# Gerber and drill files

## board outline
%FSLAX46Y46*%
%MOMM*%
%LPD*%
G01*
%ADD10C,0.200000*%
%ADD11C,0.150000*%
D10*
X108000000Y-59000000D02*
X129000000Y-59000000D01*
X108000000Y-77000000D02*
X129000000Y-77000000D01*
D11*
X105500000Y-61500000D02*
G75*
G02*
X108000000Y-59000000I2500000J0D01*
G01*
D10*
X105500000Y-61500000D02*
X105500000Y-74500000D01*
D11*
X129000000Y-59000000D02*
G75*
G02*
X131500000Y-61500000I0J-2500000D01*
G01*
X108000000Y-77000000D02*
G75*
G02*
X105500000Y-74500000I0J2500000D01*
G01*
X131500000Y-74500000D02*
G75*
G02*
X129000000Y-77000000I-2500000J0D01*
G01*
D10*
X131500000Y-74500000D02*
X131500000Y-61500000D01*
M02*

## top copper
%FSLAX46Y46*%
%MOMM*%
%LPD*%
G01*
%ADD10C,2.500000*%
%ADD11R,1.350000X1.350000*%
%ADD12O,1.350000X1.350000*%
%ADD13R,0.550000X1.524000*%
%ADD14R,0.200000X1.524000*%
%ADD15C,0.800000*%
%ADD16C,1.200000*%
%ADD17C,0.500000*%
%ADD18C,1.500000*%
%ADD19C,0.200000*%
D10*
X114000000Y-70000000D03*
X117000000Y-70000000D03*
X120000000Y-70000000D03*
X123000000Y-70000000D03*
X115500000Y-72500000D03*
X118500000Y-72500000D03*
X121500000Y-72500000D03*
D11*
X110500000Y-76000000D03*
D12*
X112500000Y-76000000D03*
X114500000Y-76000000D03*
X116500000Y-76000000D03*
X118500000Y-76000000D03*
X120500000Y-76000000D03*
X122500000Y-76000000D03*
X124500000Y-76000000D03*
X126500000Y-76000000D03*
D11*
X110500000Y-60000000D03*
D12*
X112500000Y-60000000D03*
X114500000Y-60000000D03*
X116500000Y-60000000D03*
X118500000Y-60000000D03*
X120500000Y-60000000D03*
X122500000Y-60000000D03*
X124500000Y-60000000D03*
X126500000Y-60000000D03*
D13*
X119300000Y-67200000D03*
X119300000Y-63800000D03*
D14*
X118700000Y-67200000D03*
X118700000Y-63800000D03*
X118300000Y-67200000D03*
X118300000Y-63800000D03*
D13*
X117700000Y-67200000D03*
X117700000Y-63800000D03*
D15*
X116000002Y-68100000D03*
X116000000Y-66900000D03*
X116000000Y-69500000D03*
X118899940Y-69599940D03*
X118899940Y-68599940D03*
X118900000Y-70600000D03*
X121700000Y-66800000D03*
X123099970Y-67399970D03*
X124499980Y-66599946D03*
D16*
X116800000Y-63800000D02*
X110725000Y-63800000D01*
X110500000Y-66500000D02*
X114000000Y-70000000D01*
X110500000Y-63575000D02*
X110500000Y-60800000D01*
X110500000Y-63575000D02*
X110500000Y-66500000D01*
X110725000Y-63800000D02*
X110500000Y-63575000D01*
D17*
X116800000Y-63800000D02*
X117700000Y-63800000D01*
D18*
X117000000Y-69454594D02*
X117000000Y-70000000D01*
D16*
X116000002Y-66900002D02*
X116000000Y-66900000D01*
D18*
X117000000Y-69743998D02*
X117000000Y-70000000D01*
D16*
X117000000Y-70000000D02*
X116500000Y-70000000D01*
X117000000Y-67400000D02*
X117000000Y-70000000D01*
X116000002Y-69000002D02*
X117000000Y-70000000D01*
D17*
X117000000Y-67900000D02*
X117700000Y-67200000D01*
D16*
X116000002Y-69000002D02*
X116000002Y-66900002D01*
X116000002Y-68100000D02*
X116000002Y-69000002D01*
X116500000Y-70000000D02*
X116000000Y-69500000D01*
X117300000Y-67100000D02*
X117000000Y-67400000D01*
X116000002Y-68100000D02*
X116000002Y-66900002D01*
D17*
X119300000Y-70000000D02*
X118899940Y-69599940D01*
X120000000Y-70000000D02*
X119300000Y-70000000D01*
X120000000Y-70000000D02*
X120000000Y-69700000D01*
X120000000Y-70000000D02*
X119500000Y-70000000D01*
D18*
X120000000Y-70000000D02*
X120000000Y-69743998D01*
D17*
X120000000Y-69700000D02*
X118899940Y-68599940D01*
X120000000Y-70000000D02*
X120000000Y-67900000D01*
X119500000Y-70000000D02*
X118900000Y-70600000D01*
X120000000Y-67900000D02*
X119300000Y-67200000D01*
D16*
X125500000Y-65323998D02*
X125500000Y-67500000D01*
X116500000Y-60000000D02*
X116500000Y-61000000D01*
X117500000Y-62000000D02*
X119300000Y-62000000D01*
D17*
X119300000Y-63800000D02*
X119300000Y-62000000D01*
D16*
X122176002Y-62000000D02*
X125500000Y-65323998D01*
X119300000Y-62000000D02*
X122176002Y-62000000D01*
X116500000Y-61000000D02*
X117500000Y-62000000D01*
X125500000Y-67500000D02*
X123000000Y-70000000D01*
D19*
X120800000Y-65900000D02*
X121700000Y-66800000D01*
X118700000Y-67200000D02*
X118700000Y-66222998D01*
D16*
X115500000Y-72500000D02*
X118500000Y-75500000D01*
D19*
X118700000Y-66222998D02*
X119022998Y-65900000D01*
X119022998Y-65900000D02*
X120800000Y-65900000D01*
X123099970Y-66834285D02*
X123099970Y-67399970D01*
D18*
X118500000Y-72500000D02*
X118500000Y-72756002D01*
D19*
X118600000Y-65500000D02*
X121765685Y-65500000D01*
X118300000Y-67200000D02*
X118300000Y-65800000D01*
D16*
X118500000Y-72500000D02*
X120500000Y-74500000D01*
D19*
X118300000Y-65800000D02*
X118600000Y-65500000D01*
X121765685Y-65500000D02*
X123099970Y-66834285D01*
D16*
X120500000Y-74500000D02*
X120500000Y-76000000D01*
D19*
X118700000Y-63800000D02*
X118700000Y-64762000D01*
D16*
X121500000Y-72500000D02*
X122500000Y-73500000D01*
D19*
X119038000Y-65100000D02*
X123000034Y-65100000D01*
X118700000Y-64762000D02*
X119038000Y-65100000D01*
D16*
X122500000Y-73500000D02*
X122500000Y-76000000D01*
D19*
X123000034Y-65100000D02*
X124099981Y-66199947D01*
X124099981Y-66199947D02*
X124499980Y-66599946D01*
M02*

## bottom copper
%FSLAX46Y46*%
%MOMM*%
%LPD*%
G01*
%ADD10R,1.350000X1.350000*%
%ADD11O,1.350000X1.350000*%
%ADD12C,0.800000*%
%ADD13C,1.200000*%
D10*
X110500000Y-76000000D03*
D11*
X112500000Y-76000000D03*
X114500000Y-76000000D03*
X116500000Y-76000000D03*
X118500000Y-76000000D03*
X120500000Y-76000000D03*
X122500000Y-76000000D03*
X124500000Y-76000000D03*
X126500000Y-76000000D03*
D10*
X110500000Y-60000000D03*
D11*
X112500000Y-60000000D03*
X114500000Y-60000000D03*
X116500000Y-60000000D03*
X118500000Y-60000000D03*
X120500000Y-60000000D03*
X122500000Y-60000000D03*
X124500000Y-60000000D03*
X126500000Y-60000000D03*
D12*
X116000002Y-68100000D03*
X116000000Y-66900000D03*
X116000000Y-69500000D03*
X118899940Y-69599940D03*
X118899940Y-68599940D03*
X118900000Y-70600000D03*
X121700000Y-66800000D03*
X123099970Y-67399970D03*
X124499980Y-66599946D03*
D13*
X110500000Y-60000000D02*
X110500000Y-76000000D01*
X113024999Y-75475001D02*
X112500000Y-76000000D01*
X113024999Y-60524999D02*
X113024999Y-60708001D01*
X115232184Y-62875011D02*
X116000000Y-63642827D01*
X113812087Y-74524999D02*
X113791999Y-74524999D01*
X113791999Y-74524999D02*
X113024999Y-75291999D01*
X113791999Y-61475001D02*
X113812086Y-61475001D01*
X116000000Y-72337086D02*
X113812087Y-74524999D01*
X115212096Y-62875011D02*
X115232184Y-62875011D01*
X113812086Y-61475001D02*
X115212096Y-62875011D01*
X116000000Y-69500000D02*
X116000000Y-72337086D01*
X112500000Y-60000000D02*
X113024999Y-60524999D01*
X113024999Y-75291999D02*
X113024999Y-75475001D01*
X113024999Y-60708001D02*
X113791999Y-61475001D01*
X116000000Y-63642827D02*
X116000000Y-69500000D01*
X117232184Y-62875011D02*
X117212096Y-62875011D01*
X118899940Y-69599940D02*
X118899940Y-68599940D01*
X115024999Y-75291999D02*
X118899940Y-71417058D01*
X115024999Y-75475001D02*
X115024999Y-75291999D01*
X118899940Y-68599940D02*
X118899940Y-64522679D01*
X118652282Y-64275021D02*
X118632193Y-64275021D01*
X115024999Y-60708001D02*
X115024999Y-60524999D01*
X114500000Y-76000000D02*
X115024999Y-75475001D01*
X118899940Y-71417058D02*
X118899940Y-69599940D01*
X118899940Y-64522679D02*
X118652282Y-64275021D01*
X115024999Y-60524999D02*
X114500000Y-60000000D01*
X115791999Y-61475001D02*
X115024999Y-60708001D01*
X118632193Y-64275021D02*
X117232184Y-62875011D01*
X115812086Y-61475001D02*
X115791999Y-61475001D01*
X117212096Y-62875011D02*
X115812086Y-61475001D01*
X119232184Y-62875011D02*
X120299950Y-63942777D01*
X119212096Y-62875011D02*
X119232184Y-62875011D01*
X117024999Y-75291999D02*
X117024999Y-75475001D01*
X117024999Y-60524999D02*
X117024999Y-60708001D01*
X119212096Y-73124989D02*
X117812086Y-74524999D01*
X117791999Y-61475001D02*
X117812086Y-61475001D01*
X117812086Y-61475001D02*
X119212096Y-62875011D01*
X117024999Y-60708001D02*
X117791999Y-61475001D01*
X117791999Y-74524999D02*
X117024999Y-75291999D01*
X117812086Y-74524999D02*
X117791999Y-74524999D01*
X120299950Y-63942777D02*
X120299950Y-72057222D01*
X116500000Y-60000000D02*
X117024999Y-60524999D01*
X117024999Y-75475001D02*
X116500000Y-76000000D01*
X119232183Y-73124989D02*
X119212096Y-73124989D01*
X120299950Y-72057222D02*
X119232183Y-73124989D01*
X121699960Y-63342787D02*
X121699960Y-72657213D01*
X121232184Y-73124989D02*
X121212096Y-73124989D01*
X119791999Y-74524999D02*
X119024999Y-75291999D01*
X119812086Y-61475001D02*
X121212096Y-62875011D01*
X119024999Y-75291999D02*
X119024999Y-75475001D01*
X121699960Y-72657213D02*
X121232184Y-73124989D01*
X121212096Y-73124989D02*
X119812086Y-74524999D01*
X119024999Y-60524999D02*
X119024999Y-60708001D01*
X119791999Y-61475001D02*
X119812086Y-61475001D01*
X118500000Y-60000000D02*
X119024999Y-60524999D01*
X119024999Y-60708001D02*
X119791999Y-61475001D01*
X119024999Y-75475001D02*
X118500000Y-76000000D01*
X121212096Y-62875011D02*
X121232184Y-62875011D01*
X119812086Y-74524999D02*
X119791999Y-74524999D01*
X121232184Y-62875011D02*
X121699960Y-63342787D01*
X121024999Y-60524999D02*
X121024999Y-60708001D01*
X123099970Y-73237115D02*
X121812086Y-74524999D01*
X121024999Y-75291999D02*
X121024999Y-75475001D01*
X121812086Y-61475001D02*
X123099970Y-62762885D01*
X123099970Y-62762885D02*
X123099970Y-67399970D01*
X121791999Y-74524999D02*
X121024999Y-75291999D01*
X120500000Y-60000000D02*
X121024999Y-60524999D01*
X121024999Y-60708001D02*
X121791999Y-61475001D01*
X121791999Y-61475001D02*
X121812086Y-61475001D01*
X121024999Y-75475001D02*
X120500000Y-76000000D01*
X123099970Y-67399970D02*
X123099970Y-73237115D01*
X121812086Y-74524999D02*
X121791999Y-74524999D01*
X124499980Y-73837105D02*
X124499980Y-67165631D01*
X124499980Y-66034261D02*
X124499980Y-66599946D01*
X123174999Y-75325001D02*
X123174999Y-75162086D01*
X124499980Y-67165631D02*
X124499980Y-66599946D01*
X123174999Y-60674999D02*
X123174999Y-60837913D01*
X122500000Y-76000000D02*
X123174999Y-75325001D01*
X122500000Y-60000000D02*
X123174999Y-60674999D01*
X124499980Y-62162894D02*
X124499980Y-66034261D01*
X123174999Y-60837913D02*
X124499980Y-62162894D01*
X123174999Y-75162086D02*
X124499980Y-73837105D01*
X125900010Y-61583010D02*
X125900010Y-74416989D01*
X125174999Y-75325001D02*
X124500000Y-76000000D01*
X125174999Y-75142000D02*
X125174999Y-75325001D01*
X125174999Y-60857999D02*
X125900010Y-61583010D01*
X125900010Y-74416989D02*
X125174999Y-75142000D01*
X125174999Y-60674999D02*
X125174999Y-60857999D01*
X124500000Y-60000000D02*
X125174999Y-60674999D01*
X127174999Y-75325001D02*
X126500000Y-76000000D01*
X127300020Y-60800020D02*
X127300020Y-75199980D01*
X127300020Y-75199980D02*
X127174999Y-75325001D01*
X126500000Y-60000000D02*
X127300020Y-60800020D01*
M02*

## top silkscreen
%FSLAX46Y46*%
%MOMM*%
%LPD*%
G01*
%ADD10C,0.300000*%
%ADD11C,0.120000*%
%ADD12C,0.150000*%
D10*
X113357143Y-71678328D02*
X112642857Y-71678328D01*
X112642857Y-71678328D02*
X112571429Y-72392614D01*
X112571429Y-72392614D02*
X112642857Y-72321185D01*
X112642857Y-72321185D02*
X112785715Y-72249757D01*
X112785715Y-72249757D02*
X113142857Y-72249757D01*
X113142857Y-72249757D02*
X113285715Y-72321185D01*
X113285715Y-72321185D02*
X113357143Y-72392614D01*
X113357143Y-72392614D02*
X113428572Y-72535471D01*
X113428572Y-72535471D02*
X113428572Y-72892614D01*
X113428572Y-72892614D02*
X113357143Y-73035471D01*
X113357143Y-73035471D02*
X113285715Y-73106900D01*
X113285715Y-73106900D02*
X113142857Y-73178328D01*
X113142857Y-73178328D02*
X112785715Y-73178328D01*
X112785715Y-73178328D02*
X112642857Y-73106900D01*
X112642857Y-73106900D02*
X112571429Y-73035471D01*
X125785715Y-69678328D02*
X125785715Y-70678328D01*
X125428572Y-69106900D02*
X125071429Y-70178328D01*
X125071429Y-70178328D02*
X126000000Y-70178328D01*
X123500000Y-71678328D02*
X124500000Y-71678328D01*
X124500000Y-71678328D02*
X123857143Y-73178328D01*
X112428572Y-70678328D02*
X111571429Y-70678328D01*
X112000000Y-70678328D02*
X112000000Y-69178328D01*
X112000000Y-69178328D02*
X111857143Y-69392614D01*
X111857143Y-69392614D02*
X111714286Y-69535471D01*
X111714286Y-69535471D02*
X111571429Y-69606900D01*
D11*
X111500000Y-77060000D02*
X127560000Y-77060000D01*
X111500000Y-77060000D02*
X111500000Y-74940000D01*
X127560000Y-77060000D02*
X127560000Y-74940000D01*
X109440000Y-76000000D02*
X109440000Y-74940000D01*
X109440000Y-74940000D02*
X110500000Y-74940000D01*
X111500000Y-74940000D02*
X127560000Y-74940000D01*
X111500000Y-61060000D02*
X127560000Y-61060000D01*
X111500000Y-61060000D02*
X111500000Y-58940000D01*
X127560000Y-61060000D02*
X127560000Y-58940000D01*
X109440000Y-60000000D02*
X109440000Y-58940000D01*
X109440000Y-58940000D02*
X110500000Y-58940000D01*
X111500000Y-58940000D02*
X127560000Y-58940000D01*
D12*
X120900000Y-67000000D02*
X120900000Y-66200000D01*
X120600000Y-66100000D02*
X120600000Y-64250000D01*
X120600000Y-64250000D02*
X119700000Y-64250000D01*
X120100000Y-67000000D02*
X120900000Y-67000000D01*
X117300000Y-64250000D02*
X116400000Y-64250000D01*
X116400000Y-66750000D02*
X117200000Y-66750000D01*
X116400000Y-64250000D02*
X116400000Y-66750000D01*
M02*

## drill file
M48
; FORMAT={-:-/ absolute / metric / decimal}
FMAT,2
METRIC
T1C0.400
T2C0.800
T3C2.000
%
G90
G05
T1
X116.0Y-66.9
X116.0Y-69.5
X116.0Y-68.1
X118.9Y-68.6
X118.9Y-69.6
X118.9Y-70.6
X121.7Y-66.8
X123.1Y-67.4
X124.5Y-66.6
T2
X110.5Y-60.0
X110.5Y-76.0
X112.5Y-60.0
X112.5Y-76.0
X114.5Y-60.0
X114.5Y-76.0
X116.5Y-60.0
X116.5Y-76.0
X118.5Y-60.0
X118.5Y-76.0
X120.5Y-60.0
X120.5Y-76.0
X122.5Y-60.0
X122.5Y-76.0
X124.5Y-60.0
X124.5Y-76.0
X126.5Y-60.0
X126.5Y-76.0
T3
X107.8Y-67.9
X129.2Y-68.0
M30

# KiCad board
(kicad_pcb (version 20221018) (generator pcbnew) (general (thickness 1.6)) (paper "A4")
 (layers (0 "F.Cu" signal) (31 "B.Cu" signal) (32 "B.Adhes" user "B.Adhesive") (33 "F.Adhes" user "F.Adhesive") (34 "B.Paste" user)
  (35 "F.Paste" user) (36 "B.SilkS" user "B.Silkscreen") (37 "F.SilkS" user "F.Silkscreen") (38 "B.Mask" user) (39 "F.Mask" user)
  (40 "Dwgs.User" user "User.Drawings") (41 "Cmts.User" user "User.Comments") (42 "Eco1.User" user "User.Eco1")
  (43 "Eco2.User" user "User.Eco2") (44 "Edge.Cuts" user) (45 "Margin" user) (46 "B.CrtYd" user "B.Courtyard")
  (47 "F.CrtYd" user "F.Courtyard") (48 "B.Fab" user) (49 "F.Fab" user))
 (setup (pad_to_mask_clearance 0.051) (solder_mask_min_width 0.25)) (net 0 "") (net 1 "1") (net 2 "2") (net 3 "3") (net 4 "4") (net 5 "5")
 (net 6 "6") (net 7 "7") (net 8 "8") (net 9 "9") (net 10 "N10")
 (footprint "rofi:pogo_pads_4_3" (layer "F.Cu") (at 118.5 70)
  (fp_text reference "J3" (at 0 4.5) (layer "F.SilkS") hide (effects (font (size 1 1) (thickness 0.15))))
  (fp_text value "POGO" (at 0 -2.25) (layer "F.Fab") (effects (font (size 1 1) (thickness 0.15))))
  (pad "1" smd circle (at -4.5 0) (size 2.5 2.5) (layers "F.Cu" "F.Paste" "F.Mask") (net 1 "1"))
  (pad "2" smd circle (at -1.5 0) (size 2.5 2.5) (layers "F.Cu" "F.Paste" "F.Mask") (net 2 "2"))
  (pad "3" smd circle (at 1.5 0) (size 2.5 2.5) (layers "F.Cu" "F.Paste" "F.Mask") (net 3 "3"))
  (pad "4" smd circle (at 4.5 0) (size 2.5 2.5) (layers "F.Cu" "F.Paste" "F.Mask") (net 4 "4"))
  (pad "5" smd circle (at -3 2.5) (size 2.5 2.5) (layers "F.Cu" "F.Paste" "F.Mask") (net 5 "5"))
  (pad "6" smd circle (at 0 2.5) (size 2.5 2.5) (layers "F.Cu" "F.Paste" "F.Mask") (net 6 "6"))
  (pad "7" smd circle (at 3 2.5) (size 2.5 2.5) (layers "F.Cu" "F.Paste" "F.Mask") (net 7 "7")))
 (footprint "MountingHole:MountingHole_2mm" (layer "F.Cu") (at 129.2 68)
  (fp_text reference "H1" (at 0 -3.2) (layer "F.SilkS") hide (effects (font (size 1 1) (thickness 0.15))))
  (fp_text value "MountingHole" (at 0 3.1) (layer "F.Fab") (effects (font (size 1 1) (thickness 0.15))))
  (pad "" np_thru_hole circle (at 0 0) (size 2 2) (drill 2) (layers "*.Cu" "*.Mask")))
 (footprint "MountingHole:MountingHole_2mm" (layer "F.Cu") (at 107.8 67.9)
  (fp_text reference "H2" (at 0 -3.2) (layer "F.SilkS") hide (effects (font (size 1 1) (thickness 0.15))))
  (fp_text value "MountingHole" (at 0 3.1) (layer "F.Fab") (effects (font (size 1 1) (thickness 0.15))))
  (pad "" np_thru_hole circle (at 0 0) (size 2 2) (drill 2) (layers "*.Cu" "*.Mask")))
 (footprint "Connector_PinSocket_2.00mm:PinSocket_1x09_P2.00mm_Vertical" (layer "F.Cu") (at 110.5 76 90)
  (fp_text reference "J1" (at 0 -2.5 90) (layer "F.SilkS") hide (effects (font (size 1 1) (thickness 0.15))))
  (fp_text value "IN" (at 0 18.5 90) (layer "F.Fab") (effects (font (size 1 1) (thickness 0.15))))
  (fp_line (start -1.06 1) (end -1.06 17.06) (stroke (width 0.12) (type solid)) (layer "F.SilkS"))
  (fp_line (start -1.06 1) (end 1.06 1) (stroke (width 0.12) (type solid)) (layer "F.SilkS"))
  (fp_line (start -1.06 17.06) (end 1.06 17.06) (stroke (width 0.12) (type solid)) (layer "F.SilkS"))
  (fp_line (start 0 -1.06) (end 1.06 -1.06) (stroke (width 0.12) (type solid)) (layer "F.SilkS"))
  (fp_line (start 1.06 -1.06) (end 1.06 0) (stroke (width 0.12) (type solid)) (layer "F.SilkS"))
  (fp_line (start 1.06 1) (end 1.06 17.06) (stroke (width 0.12) (type solid)) (layer "F.SilkS"))
  (pad "1" thru_hole rect (at 0 0 90) (size 1.35 1.35) (drill 0.8) (layers "*.Cu" "*.Mask") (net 1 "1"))
  (pad "2" thru_hole oval (at 0 2 90) (size 1.35 1.35) (drill 0.8) (layers "*.Cu" "*.Mask") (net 2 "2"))
  (pad "3" thru_hole oval (at 0 4 90) (size 1.35 1.35) (drill 0.8) (layers "*.Cu" "*.Mask") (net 3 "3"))
  (pad "4" thru_hole oval (at 0 6 90) (size 1.35 1.35) (drill 0.8) (layers "*.Cu" "*.Mask") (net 4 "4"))
  (pad "5" thru_hole oval (at 0 8 90) (size 1.35 1.35) (drill 0.8) (layers "*.Cu" "*.Mask") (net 5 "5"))
  (pad "6" thru_hole oval (at 0 10 90) (size 1.35 1.35) (drill 0.8) (layers "*.Cu" "*.Mask") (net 6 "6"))
  (pad "7" thru_hole oval (at 0 12 90) (size 1.35 1.35) (drill 0.8) (layers "*.Cu" "*.Mask") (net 7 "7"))
  (pad "8" thru_hole oval (at 0 14 90) (size 1.35 1.35) (drill 0.8) (layers "*.Cu" "*.Mask") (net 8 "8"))
  (pad "9" thru_hole oval (at 0 16 90) (size 1.35 1.35) (drill 0.8) (layers "*.Cu" "*.Mask") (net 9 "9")))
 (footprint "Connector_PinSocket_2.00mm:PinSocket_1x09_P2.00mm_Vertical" (layer "F.Cu") (at 110.5 60 90)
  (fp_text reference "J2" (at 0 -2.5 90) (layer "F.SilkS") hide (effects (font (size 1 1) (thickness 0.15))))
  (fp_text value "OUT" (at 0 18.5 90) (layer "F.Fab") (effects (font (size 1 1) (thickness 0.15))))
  (fp_line (start -1.06 1) (end -1.06 17.06) (stroke (width 0.12) (type solid)) (layer "F.SilkS"))
  (fp_line (start -1.06 1) (end 1.06 1) (stroke (width 0.12) (type solid)) (layer "F.SilkS"))
  (fp_line (start -1.06 17.06) (end 1.06 17.06) (stroke (width 0.12) (type solid)) (layer "F.SilkS"))
  (fp_line (start 0 -1.06) (end 1.06 -1.06) (stroke (width 0.12) (type solid)) (layer "F.SilkS"))
  (fp_line (start 1.06 -1.06) (end 1.06 0) (stroke (width 0.12) (type solid)) (layer "F.SilkS"))
  (fp_line (start 1.06 1) (end 1.06 17.06) (stroke (width 0.12) (type solid)) (layer "F.SilkS"))
  (pad "1" thru_hole rect (at 0 0 90) (size 1.35 1.35) (drill 0.8) (layers "*.Cu" "*.Mask") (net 1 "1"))
  (pad "2" thru_hole oval (at 0 2 90) (size 1.35 1.35) (drill 0.8) (layers "*.Cu" "*.Mask") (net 2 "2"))
  (pad "3" thru_hole oval (at 0 4 90) (size 1.35 1.35) (drill 0.8) (layers "*.Cu" "*.Mask") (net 3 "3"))
  (pad "4" thru_hole oval (at 0 6 90) (size 1.35 1.35) (drill 0.8) (layers "*.Cu" "*.Mask") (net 4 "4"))
  (pad "5" thru_hole oval (at 0 8 90) (size 1.35 1.35) (drill 0.8) (layers "*.Cu" "*.Mask") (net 5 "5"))
  (pad "6" thru_hole oval (at 0 10 90) (size 1.35 1.35) (drill 0.8) (layers "*.Cu" "*.Mask") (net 6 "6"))
  (pad "7" thru_hole oval (at 0 12 90) (size 1.35 1.35) (drill 0.8) (layers "*.Cu" "*.Mask") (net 7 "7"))
  (pad "8" thru_hole oval (at 0 14 90) (size 1.35 1.35) (drill 0.8) (layers "*.Cu" "*.Mask") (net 8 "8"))
  (pad "9" thru_hole oval (at 0 16 90) (size 1.35 1.35) (drill 0.8) (layers "*.Cu" "*.Mask") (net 9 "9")))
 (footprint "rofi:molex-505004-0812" (layer "F.Cu") (at 118.5 65.5 180)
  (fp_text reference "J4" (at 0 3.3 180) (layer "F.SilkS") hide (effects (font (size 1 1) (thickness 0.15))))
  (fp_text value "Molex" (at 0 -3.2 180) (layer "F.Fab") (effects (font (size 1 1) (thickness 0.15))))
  (fp_line (start -2.4 -1.5) (end -2.4 -0.7) (stroke (width 0.15) (type solid)) (layer "F.SilkS"))
  (fp_line (start -2.1 -0.6) (end -2.1 1.25) (stroke (width 0.15) (type solid)) (layer "F.SilkS"))
  (fp_line (start -2.1 1.25) (end -1.2 1.25) (stroke (width 0.15) (type solid)) (layer "F.SilkS"))
  (fp_line (start -1.6 -1.5) (end -2.4 -1.5) (stroke (width 0.15) (type solid)) (layer "F.SilkS"))
  (fp_line (start 1.2 1.25) (end 2.1 1.25) (stroke (width 0.15) (type solid)) (layer "F.SilkS"))
  (fp_line (start 2.1 -1.25) (end 1.3 -1.25) (stroke (width 0.15) (type solid)) (layer "F.SilkS"))
  (fp_line (start 2.1 1.25) (end 2.1 -1.25) (stroke (width 0.15) (type solid)) (layer "F.SilkS"))
  (pad "1" smd rect (at -0.8 -1.7 180) (size 0.55 1.524) (layers "F.Cu" "F.Paste" "F.Mask") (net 3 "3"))
  (pad "2" smd rect (at -0.8 1.7 180) (size 0.55 1.524) (layers "F.Cu" "F.Paste" "F.Mask") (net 4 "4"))
  (pad "3" smd rect (at -0.2 -1.7 180) (size 0.2 1.524) (layers "F.Cu" "F.Paste" "F.Mask") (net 5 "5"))
  (pad "4" smd rect (at -0.2 1.7 180) (size 0.2 1.524) (layers "F.Cu" "F.Paste" "F.Mask") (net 7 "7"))
  (pad "5" smd rect (at 0.2 -1.7 180) (size 0.2 1.524) (layers "F.Cu" "F.Paste" "F.Mask") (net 6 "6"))
  (pad "6" smd rect (at 0.2 1.7 180) (size 0.2 1.524) (layers "F.Cu" "F.Paste" "F.Mask") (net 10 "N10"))
  (pad "7" smd rect (at 0.8 -1.7 180) (size 0.55 1.524) (layers "F.Cu" "F.Paste" "F.Mask") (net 2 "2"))
  (pad "8" smd rect (at 0.8 1.7 180) (size 0.55 1.524) (layers "F.Cu" "F.Paste" "F.Mask") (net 1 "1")))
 (gr_line (start 108 59) (end 129 59) (stroke (width 0.2) (type solid)) (layer "Edge.Cuts"))
 (gr_line (start 108 77) (end 129 77) (stroke (width 0.2) (type solid)) (layer "Edge.Cuts"))
 (gr_arc (start 105.5 61.5) (mid 106.232233 59.732233) (end 108 59) (stroke (width 0.15) (type solid)) (layer "Edge.Cuts"))
 (gr_line (start 105.5 61.5) (end 105.5 74.5) (stroke (width 0.2) (type solid)) (layer "Edge.Cuts"))
 (gr_arc (start 129 59) (mid 130.767767 59.732233) (end 131.5 61.5) (stroke (width 0.15) (type solid)) (layer "Edge.Cuts"))
 (gr_arc (start 108 77) (mid 106.232233 76.267767) (end 105.5 74.5) (stroke (width 0.15) (type solid)) (layer "Edge.Cuts"))
 (gr_arc (start 131.5 74.5) (mid 130.767767 76.267767) (end 129 77) (stroke (width 0.15) (type solid)) (layer "Edge.Cuts"))
 (gr_line (start 131.5 74.5) (end 131.5 61.5) (stroke (width 0.2) (type solid)) (layer "Edge.Cuts"))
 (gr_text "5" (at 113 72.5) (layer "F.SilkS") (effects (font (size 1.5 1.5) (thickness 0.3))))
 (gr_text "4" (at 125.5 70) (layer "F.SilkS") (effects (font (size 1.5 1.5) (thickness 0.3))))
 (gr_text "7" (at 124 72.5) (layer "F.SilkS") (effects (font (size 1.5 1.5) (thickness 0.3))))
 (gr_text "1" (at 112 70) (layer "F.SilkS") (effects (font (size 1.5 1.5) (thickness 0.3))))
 (segment (start 116.8 63.8) (end 110.725 63.8) (width 1.2) (layer "F.Cu") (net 1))
 (segment (start 110.5 66.5) (end 114 70) (width 1.2) (layer "F.Cu") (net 1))
 (segment (start 110.5 63.575) (end 110.5 60.8) (width 1.2) (layer "F.Cu") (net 1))
 (segment (start 110.5 63.575) (end 110.5 66.5) (width 1.2) (layer "F.Cu") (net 1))
 (segment (start 110.725 63.8) (end 110.5 63.575) (width 1.2) (layer "F.Cu") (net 1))
 (segment (start 116.8 63.8) (end 117.7 63.8) (width 0.5) (layer "F.Cu") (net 1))
 (segment (start 110.5 60) (end 110.5 76) (width 1.2) (layer "B.Cu") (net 1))
 (segment (start 117 69.454594) (end 117 70) (width 1.5) (layer "F.Cu") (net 2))
 (segment (start 116.000002 66.900002) (end 116 66.9) (width 1.2) (layer "F.Cu") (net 2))
 (segment (start 117 69.743998) (end 117 70) (width 1.5) (layer "F.Cu") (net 2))
 (segment (start 117 70) (end 116.5 70) (width 1.2) (layer "F.Cu") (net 2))
 (segment (start 117 67.4) (end 117 70) (width 1.2) (layer "F.Cu") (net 2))
 (segment (start 116.000002 69.000002) (end 117 70) (width 1.2) (layer "F.Cu") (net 2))
 (segment (start 117 67.9) (end 117.7 67.2) (width 0.5) (layer "F.Cu") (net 2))
 (segment (start 116.000002 69.000002) (end 116.000002 66.900002) (width 1.2) (layer "F.Cu") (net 2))
 (segment (start 116.000002 68.1) (end 116.000002 69.000002) (width 1.2) (layer "F.Cu") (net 2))
 (segment (start 116.5 70) (end 116 69.5) (width 1.2) (layer "F.Cu") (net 2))
 (segment (start 117.3 67.1) (end 117 67.4) (width 1.2) (layer "F.Cu") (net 2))
 (segment (start 116.000002 68.1) (end 116.000002 66.900002) (width 1.2) (layer "F.Cu") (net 2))
 (via (at 116.000002 68.1) (size 0.8) (drill 0.4) (layers "F.Cu" "B.Cu") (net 2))
 (via (at 116 66.9) (size 0.8) (drill 0.4) (layers "F.Cu" "B.Cu") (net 2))
 (via (at 116 69.5) (size 0.8) (drill 0.4) (layers "F.Cu" "B.Cu") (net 2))
 (segment (start 113.024999 75.475001) (end 112.5 76) (width 1.2) (layer "B.Cu") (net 2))
 (segment (start 113.024999 60.524999) (end 113.024999 60.708001) (width 1.2) (layer "B.Cu") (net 2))
 (segment (start 115.232184 62.875011) (end 116 63.642827) (width 1.2) (layer "B.Cu") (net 2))
 (segment (start 113.812087 74.524999) (end 113.791999 74.524999) (width 1.2) (layer "B.Cu") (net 2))
 (segment (start 113.791999 74.524999) (end 113.024999 75.291999) (width 1.2) (layer "B.Cu") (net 2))
 (segment (start 113.791999 61.475001) (end 113.812086 61.475001) (width 1.2) (layer "B.Cu") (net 2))
 (segment (start 116 72.337086) (end 113.812087 74.524999) (width 1.2) (layer "B.Cu") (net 2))
 (segment (start 115.212096 62.875011) (end 115.232184 62.875011) (width 1.2) (layer "B.Cu") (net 2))
 (segment (start 113.812086 61.475001) (end 115.212096 62.875011) (width 1.2) (layer "B.Cu") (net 2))
 (segment (start 116 69.5) (end 116 72.337086) (width 1.2) (layer "B.Cu") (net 2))
 (segment (start 112.5 60) (end 113.024999 60.524999) (width 1.2) (layer "B.Cu") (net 2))
 (segment (start 113.024999 75.291999) (end 113.024999 75.475001) (width 1.2) (layer "B.Cu") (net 2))
 (segment (start 113.024999 60.708001) (end 113.791999 61.475001) (width 1.2) (layer "B.Cu") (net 2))
 (segment (start 116 63.642827) (end 116 69.5) (width 1.2) (layer "B.Cu") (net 2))
 (segment (start 119.3 70) (end 118.89994 69.59994) (width 0.5) (layer "F.Cu") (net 3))
 (segment (start 120 70) (end 119.3 70) (width 0.5) (layer "F.Cu") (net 3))
 (segment (start 120 70) (end 120 69.7) (width 0.5) (layer "F.Cu") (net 3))
 (segment (start 120 70) (end 119.5 70) (width 0.5) (layer "F.Cu") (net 3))
 (segment (start 120 70) (end 120 69.743998) (width 1.5) (layer "F.Cu") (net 3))
 (segment (start 120 69.7) (end 118.89994 68.59994) (width 0.5) (layer "F.Cu") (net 3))
 (segment (start 120 70) (end 120 67.9) (width 0.5) (layer "F.Cu") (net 3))
 (segment (start 119.5 70) (end 118.9 70.6) (width 0.5) (layer "F.Cu") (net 3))
 (segment (start 120 67.9) (end 119.3 67.2) (width 0.5) (layer "F.Cu") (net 3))
 (via (at 118.89994 69.59994) (size 0.8) (drill 0.4) (layers "F.Cu" "B.Cu") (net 3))
 (via (at 118.89994 68.59994) (size 0.8) (drill 0.4) (layers "F.Cu" "B.Cu") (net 3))
 (via (at 118.9 70.6) (size 0.8) (drill 0.4) (layers "F.Cu" "B.Cu") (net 3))
 (segment (start 117.232184 62.875011) (end 117.212096 62.875011) (width 1.2) (layer "B.Cu") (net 3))
 (segment (start 118.89994 69.59994) (end 118.89994 68.59994) (width 1.2) (layer "B.Cu") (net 3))
 (segment (start 115.024999 75.291999) (end 118.89994 71.417058) (width 1.2) (layer "B.Cu") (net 3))
 (segment (start 115.024999 75.475001) (end 115.024999 75.291999) (width 1.2) (layer "B.Cu") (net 3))
 (segment (start 118.89994 68.59994) (end 118.89994 64.522679) (width 1.2) (layer "B.Cu") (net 3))
 (segment (start 118.652282 64.275021) (end 118.632193 64.275021) (width 1.2) (layer "B.Cu") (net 3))
 (segment (start 115.024999 60.708001) (end 115.024999 60.524999) (width 1.2) (layer "B.Cu") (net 3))
 (segment (start 114.5 76) (end 115.024999 75.475001) (width 1.2) (layer "B.Cu") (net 3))
 (segment (start 118.89994 71.417058) (end 118.89994 69.59994) (width 1.2) (layer "B.Cu") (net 3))
 (segment (start 118.89994 64.522679) (end 118.652282 64.275021) (width 1.2) (layer "B.Cu") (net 3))
 (segment (start 115.024999 60.524999) (end 114.5 60) (width 1.2) (layer "B.Cu") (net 3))
 (segment (start 115.791999 61.475001) (end 115.024999 60.708001) (width 1.2) (layer "B.Cu") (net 3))
 (segment (start 118.632193 64.275021) (end 117.232184 62.875011) (width 1.2) (layer "B.Cu") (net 3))
 (segment (start 115.812086 61.475001) (end 115.791999 61.475001) (width 1.2) (layer "B.Cu") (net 3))
 (segment (start 117.212096 62.875011) (end 115.812086 61.475001) (width 1.2) (layer "B.Cu") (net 3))
 (segment (start 125.5 65.323998) (end 125.5 67.5) (width 1.2) (layer "F.Cu") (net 4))
 (segment (start 116.5 60) (end 116.5 61) (width 1.2) (layer "F.Cu") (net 4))
 (segment (start 117.5 62) (end 119.3 62) (width 1.2) (layer "F.Cu") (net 4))
 (segment (start 119.3 63.8) (end 119.3 62) (width 0.5) (layer "F.Cu") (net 4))
 (segment (start 122.176002 62) (end 125.5 65.323998) (width 1.2) (layer "F.Cu") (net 4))
 (segment (start 119.3 62) (end 122.176002 62) (width 1.2) (layer "F.Cu") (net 4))
 (segment (start 116.5 61) (end 117.5 62) (width 1.2) (layer "F.Cu") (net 4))
 (segment (start 125.5 67.5) (end 123 70) (width 1.2) (layer "F.Cu") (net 4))
 (segment (start 119.232184 62.875011) (end 120.29995 63.942777) (width 1.2) (layer "B.Cu") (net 4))
 (segment (start 119.212096 62.875011) (end 119.232184 62.875011) (width 1.2) (layer "B.Cu") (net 4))
 (segment (start 117.024999 75.291999) (end 117.024999 75.475001) (width 1.2) (layer "B.Cu") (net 4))
 (segment (start 117.024999 60.524999) (end 117.024999 60.708001) (width 1.2) (layer "B.Cu") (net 4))
 (segment (start 119.212096 73.124989) (end 117.812086 74.524999) (width 1.2) (layer "B.Cu") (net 4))
 (segment (start 117.791999 61.475001) (end 117.812086 61.475001) (width 1.2) (layer "B.Cu") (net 4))
 (segment (start 117.812086 61.475001) (end 119.212096 62.875011) (width 1.2) (layer "B.Cu") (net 4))
 (segment (start 117.024999 60.708001) (end 117.791999 61.475001) (width 1.2) (layer "B.Cu") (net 4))
 (segment (start 117.791999 74.524999) (end 117.024999 75.291999) (width 1.2) (layer "B.Cu") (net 4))
 (segment (start 117.812086 74.524999) (end 117.791999 74.524999) (width 1.2) (layer "B.Cu") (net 4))
 (segment (start 120.29995 63.942777) (end 120.29995 72.057222) (width 1.2) (layer "B.Cu") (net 4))
 (segment (start 116.5 60) (end 117.024999 60.524999) (width 1.2) (layer "B.Cu") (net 4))
 (segment (start 117.024999 75.475001) (end 116.5 76) (width 1.2) (layer "B.Cu") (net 4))
 (segment (start 119.232183 73.124989) (end 119.212096 73.124989) (width 1.2) (layer "B.Cu") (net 4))
 (segment (start 120.29995 72.057222) (end 119.232183 73.124989) (width 1.2) (layer "B.Cu") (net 4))
 (segment (start 120.8 65.9) (end 121.7 66.8) (width 0.2) (layer "F.Cu") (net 5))
 (segment (start 118.7 67.2) (end 118.7 66.222998) (width 0.2) (layer "F.Cu") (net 5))
 (segment (start 115.5 72.5) (end 118.5 75.5) (width 1.2) (layer "F.Cu") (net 5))
 (segment (start 118.7 66.222998) (end 119.022998 65.9) (width 0.2) (layer "F.Cu") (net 5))
 (segment (start 119.022998 65.9) (end 120.8 65.9) (width 0.2) (layer "F.Cu") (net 5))
 (via (at 121.7 66.8) (size 0.8) (drill 0.4) (layers "F.Cu" "B.Cu") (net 5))
 (segment (start 121.69996 63.342787) (end 121.69996 72.657213) (width 1.2) (layer "B.Cu") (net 5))
 (segment (start 121.232184 73.124989) (end 121.212096 73.124989) (width 1.2) (layer "B.Cu") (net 5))
 (segment (start 119.791999 74.524999) (end 119.024999 75.291999) (width 1.2) (layer "B.Cu") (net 5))
 (segment (start 119.812086 61.475001) (end 121.212096 62.875011) (width 1.2) (layer "B.Cu") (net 5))
 (segment (start 119.024999 75.291999) (end 119.024999 75.475001) (width 1.2) (layer "B.Cu") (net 5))
 (segment (start 121.69996 72.657213) (end 121.232184 73.124989) (width 1.2) (layer "B.Cu") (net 5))
 (segment (start 121.212096 73.124989) (end 119.812086 74.524999) (width 1.2) (layer "B.Cu") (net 5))
 (segment (start 119.024999 60.524999) (end 119.024999 60.708001) (width 1.2) (layer "B.Cu") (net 5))
 (segment (start 119.791999 61.475001) (end 119.812086 61.475001) (width 1.2) (layer "B.Cu") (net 5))
 (segment (start 118.5 60) (end 119.024999 60.524999) (width 1.2) (layer "B.Cu") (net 5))
 (segment (start 119.024999 60.708001) (end 119.791999 61.475001) (width 1.2) (layer "B.Cu") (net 5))
 (segment (start 119.024999 75.475001) (end 118.5 76) (width 1.2) (layer "B.Cu") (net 5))
 (segment (start 121.212096 62.875011) (end 121.232184 62.875011) (width 1.2) (layer "B.Cu") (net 5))
 (segment (start 119.812086 74.524999) (end 119.791999 74.524999) (width 1.2) (layer "B.Cu") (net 5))
 (segment (start 121.232184 62.875011) (end 121.69996 63.342787) (width 1.2) (layer "B.Cu") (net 5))
 (segment (start 123.09997 66.834285) (end 123.09997 67.39997) (width 0.2) (layer "F.Cu") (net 6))
 (segment (start 118.5 72.5) (end 118.5 72.756002) (width 1.5) (layer "F.Cu") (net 6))
 (segment (start 118.6 65.5) (end 121.765685 65.5) (width 0.2) (layer "F.Cu") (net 6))
 (segment (start 118.3 67.2) (end 118.3 65.8) (width 0.2) (layer "F.Cu") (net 6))
 (segment (start 118.5 72.5) (end 120.5 74.5) (width 1.2) (layer "F.Cu") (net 6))
 (segment (start 118.3 65.8) (end 118.6 65.5) (width 0.2) (layer "F.Cu") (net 6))
 (segment (start 121.765685 65.5) (end 123.09997 66.834285) (width 0.2) (layer "F.Cu") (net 6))
 (segment (start 120.5 74.5) (end 120.5 76) (width 1.2) (layer "F.Cu") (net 6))
 (via (at 123.09997 67.39997) (size 0.8) (drill 0.4) (layers "F.Cu" "B.Cu") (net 6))
 (segment (start 121.024999 60.524999) (end 121.024999 60.708001) (width 1.2) (layer "B.Cu") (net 6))
 (segment (start 123.09997 73.237115) (end 121.812086 74.524999) (width 1.2) (layer "B.Cu") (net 6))
 (segment (start 121.024999 75.291999) (end 121.024999 75.475001) (width 1.2) (layer "B.Cu") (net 6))
 (segment (start 121.812086 61.475001) (end 123.09997 62.762885) (width 1.2) (layer "B.Cu") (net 6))
 (segment (start 123.09997 62.762885) (end 123.09997 67.39997) (width 1.2) (layer "B.Cu") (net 6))
 (segment (start 121.791999 74.524999) (end 121.024999 75.291999) (width 1.2) (layer "B.Cu") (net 6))
 (segment (start 120.5 60) (end 121.024999 60.524999) (width 1.2) (layer "B.Cu") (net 6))
 (segment (start 121.024999 60.708001) (end 121.791999 61.475001) (width 1.2) (layer "B.Cu") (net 6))
 (segment (start 121.791999 61.475001) (end 121.812086 61.475001) (width 1.2) (layer "B.Cu") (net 6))
 (segment (start 121.024999 75.475001) (end 120.5 76) (width 1.2) (layer "B.Cu") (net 6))
 (segment (start 123.09997 67.39997) (end 123.09997 73.237115) (width 1.2) (layer "B.Cu") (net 6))
 (segment (start 121.812086 74.524999) (end 121.791999 74.524999) (width 1.2) (layer "B.Cu") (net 6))
 (segment (start 118.7 63.8) (end 118.7 64.762) (width 0.2) (layer "F.Cu") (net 7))
 (segment (start 121.5 72.5) (end 122.5 73.5) (width 1.2) (layer "F.Cu") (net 7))
 (segment (start 119.038 65.1) (end 123.000034 65.1) (width 0.2) (layer "F.Cu") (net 7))
 (segment (start 118.7 64.762) (end 119.038 65.1) (width 0.2) (layer "F.Cu") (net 7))
 (segment (start 122.5 73.5) (end 122.5 76) (width 1.2) (layer "F.Cu") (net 7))
 (segment (start 123.000034 65.1) (end 124.099981 66.199947) (width 0.2) (layer "F.Cu") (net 7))
 (segment (start 124.099981 66.199947) (end 124.49998 66.599946) (width 0.2) (layer "F.Cu") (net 7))
 (via (at 124.49998 66.599946) (size 0.8) (drill 0.4) (layers "F.Cu" "B.Cu") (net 7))
 (segment (start 124.49998 73.837105) (end 124.49998 67.165631) (width 1.2) (layer "B.Cu") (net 7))
 (segment (start 124.49998 66.034261) (end 124.49998 66.599946) (width 1.2) (layer "B.Cu") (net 7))
 (segment (start 123.174999 75.325001) (end 123.174999 75.162086) (width 1.2) (layer "B.Cu") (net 7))
 (segment (start 124.49998 67.165631) (end 124.49998 66.599946) (width 1.2) (layer "B.Cu") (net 7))
 (segment (start 123.174999 60.674999) (end 123.174999 60.837913) (width 1.2) (layer "B.Cu") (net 7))
 (segment (start 122.5 76) (end 123.174999 75.325001) (width 1.2) (layer "B.Cu") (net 7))
 (segment (start 122.5 60) (end 123.174999 60.674999) (width 1.2) (layer "B.Cu") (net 7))
 (segment (start 124.49998 62.162894) (end 124.49998 66.034261) (width 1.2) (layer "B.Cu") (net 7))
 (segment (start 123.174999 60.837913) (end 124.49998 62.162894) (width 1.2) (layer "B.Cu") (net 7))
 (segment (start 123.174999 75.162086) (end 124.49998 73.837105) (width 1.2) (layer "B.Cu") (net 7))
 (segment (start 125.90001 61.58301) (end 125.90001 74.416989) (width 1.2) (layer "B.Cu") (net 8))
 (segment (start 125.174999 75.325001) (end 124.5 76) (width 1.2) (layer "B.Cu") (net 8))
 (segment (start 125.174999 75.142) (end 125.174999 75.325001) (width 1.2) (layer "B.Cu") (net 8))
 (segment (start 125.174999 60.857999) (end 125.90001 61.58301) (width 1.2) (layer "B.Cu") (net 8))
 (segment (start 125.90001 74.416989) (end 125.174999 75.142) (width 1.2) (layer "B.Cu") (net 8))
 (segment (start 125.174999 60.674999) (end 125.174999 60.857999) (width 1.2) (layer "B.Cu") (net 8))
 (segment (start 124.5 60) (end 125.174999 60.674999) (width 1.2) (layer "B.Cu") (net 8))
 (segment (start 127.174999 75.325001) (end 126.5 76) (width 1.2) (layer "B.Cu") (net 9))
 (segment (start 127.30002 60.80002) (end 127.30002 75.19998) (width 1.2) (layer "B.Cu") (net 9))
 (segment (start 127.30002 75.19998) (end 127.174999 75.325001) (width 1.2) (layer "B.Cu") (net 9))
 (segment (start 126.5 60) (end 127.30002 60.80002) (width 1.2) (layer "B.Cu") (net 9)))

